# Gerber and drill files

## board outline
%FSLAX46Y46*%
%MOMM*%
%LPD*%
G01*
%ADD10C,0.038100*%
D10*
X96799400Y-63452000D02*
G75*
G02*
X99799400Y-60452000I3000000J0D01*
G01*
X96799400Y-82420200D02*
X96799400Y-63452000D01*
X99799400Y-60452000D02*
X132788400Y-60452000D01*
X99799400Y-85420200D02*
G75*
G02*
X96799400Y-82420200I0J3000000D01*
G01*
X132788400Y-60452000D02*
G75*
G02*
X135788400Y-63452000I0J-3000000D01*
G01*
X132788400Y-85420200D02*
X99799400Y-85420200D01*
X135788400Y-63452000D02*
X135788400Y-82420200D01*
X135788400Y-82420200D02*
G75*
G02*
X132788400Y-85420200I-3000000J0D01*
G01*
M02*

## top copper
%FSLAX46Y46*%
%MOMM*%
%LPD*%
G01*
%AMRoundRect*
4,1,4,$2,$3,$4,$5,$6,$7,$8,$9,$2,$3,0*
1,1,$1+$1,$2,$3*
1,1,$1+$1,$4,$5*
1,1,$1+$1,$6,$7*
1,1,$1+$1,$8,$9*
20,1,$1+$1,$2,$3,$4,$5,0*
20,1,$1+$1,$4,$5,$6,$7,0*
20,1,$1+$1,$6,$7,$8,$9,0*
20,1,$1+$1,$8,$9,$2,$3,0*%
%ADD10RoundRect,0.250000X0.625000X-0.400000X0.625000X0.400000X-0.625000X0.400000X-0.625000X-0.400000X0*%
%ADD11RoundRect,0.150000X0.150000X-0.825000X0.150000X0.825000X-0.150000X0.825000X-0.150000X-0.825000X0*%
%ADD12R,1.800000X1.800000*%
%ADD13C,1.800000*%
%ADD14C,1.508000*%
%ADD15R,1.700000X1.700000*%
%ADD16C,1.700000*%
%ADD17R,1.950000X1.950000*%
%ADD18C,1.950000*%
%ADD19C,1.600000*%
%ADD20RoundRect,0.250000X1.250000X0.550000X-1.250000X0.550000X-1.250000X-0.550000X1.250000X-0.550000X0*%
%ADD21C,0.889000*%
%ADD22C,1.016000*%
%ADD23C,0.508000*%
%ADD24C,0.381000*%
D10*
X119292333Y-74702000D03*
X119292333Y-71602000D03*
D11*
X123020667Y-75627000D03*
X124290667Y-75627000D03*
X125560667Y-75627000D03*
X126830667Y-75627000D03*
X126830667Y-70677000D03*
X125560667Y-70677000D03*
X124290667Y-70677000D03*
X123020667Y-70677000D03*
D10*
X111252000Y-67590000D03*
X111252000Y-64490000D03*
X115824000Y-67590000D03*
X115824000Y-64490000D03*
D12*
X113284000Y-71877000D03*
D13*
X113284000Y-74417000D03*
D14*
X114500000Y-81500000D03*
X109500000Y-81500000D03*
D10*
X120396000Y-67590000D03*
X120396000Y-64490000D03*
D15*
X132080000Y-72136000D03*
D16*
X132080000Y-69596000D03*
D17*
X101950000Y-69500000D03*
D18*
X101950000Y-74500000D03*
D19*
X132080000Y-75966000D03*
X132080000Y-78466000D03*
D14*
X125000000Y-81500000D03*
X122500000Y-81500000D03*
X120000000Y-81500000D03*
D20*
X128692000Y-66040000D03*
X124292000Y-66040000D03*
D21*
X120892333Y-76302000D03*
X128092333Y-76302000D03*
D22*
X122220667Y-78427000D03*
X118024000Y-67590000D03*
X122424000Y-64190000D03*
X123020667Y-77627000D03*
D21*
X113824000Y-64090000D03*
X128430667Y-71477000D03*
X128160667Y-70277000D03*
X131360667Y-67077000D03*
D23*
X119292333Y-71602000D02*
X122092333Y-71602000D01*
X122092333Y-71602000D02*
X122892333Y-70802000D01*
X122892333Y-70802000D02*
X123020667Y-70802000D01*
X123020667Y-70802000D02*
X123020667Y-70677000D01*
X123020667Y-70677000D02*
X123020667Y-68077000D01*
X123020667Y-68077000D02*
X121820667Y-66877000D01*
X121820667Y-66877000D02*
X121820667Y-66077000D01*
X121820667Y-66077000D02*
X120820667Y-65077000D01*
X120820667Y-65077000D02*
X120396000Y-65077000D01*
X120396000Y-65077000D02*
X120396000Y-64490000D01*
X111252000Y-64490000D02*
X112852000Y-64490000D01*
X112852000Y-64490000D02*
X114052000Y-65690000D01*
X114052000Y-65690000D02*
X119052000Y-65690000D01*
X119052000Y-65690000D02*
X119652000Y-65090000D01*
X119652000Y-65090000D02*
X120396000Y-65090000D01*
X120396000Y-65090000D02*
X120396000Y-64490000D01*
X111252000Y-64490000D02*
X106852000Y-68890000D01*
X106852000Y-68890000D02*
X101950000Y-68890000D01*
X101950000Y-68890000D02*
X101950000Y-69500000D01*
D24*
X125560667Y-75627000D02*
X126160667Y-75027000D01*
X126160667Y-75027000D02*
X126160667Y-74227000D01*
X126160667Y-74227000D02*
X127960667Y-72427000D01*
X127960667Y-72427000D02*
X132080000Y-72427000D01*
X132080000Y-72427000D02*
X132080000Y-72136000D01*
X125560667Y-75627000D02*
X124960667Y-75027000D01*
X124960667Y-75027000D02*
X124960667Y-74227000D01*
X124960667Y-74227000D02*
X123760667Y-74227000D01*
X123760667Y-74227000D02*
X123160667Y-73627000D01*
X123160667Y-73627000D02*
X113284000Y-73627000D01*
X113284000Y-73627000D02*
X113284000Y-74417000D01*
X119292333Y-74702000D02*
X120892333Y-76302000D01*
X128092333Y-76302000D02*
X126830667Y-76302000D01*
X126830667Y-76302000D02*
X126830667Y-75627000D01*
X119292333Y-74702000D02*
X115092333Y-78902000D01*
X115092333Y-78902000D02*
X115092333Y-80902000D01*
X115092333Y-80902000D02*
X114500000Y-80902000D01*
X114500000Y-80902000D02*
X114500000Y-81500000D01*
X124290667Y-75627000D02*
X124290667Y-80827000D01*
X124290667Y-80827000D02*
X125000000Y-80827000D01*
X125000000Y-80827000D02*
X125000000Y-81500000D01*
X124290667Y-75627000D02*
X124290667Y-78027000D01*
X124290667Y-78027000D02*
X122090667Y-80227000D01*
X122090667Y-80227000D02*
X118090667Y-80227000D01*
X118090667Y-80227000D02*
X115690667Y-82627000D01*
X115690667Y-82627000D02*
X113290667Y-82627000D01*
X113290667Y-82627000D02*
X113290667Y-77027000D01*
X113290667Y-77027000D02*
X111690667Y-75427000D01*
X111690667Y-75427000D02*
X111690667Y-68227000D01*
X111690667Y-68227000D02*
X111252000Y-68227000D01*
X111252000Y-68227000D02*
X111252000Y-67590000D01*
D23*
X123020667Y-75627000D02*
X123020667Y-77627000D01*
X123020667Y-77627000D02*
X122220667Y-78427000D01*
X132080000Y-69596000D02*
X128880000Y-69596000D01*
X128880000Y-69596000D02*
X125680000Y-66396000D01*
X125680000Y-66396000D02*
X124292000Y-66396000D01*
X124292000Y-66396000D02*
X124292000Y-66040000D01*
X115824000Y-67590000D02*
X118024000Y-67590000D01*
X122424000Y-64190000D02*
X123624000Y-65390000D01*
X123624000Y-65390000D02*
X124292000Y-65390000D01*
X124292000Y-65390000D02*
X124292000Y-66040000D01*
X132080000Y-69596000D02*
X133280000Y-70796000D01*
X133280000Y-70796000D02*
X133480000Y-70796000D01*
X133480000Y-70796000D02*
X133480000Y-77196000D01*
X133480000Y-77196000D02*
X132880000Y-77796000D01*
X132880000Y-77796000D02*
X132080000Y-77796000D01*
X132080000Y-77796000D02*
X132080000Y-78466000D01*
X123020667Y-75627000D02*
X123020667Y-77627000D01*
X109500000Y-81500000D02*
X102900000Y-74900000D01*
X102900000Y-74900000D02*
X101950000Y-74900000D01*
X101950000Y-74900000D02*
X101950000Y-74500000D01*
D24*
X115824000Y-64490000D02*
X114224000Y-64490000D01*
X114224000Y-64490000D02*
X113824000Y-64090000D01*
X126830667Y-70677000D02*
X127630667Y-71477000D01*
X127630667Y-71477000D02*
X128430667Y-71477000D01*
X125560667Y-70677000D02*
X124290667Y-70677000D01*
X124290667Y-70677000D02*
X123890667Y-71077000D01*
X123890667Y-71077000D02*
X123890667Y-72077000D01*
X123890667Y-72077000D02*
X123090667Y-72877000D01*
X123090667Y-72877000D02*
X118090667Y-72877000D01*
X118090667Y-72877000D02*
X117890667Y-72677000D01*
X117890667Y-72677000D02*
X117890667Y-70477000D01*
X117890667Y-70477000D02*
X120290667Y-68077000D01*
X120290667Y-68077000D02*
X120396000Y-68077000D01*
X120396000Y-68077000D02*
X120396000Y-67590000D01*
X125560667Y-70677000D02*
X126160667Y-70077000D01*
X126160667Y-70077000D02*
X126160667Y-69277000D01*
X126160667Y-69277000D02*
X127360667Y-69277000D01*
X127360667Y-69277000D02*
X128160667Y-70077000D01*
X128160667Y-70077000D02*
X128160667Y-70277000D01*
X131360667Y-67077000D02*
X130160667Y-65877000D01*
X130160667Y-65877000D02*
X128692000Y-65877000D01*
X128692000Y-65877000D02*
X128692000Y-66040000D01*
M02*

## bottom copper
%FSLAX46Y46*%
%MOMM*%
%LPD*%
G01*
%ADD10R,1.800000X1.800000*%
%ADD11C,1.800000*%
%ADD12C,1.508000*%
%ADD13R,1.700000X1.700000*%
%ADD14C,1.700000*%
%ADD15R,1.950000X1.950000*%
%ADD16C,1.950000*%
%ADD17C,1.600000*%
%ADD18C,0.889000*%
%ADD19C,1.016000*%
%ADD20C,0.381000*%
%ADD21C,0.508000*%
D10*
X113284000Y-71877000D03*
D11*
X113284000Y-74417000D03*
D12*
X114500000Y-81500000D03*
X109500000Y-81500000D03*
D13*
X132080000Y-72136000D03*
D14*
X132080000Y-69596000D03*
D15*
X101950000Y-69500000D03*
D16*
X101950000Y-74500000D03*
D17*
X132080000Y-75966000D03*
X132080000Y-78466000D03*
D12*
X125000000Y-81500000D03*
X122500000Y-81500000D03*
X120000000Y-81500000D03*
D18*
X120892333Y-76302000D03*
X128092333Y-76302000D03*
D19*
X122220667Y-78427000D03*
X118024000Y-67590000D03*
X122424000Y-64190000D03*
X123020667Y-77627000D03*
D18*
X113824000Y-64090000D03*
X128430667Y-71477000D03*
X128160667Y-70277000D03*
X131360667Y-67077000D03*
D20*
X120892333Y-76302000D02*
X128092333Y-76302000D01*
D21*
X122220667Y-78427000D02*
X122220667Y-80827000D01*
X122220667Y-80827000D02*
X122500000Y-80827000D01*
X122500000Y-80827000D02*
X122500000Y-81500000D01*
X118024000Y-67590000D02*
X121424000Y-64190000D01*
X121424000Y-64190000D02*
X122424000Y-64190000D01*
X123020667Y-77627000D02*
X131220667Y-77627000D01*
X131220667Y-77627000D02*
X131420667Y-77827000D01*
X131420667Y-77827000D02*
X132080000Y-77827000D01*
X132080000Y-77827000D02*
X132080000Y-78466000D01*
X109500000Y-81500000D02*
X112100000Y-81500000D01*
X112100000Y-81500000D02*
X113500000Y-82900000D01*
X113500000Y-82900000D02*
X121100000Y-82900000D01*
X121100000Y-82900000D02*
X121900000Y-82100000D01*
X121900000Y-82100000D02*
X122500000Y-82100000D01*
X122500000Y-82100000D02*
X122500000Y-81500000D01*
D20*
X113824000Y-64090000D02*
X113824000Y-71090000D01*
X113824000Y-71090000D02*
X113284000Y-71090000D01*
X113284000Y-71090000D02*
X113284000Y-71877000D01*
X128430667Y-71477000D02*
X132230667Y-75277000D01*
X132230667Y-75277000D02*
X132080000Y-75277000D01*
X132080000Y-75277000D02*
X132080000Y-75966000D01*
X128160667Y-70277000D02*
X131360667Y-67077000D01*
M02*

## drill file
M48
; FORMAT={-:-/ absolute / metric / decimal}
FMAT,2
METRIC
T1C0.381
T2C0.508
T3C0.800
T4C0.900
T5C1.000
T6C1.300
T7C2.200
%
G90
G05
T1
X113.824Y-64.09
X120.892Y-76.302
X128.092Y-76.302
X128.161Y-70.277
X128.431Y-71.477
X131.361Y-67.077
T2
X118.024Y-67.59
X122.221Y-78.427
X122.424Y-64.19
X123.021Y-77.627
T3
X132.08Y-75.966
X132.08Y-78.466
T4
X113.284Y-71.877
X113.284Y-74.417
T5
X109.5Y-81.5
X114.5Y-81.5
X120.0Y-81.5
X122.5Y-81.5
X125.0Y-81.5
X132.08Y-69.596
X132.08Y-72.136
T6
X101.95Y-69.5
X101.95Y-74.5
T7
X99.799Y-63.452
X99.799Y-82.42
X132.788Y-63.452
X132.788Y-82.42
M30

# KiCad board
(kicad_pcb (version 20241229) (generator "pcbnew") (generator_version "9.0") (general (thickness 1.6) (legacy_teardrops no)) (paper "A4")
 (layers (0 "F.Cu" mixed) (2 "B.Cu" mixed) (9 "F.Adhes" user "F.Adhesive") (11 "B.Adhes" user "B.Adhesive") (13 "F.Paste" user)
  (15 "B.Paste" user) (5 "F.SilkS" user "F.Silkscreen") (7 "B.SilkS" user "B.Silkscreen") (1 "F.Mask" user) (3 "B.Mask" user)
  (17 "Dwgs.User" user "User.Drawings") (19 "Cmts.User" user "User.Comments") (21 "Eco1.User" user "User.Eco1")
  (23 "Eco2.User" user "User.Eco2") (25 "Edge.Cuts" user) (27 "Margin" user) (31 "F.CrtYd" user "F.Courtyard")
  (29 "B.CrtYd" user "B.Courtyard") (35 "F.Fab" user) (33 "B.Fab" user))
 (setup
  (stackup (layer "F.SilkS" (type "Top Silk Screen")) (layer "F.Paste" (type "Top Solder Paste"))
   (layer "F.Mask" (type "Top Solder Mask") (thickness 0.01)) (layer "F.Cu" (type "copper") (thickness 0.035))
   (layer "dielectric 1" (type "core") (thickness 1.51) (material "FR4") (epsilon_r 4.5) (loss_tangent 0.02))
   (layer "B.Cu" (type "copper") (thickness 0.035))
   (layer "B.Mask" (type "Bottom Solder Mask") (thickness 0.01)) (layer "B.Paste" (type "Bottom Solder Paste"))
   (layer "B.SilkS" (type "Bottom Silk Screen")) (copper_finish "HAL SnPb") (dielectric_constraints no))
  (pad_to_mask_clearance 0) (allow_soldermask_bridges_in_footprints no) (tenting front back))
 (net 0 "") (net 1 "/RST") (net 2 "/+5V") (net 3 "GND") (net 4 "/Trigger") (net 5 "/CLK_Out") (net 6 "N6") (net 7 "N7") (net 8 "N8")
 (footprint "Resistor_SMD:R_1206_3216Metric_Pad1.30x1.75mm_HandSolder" (layer "F.Cu") (at 119.292333 73.152 90)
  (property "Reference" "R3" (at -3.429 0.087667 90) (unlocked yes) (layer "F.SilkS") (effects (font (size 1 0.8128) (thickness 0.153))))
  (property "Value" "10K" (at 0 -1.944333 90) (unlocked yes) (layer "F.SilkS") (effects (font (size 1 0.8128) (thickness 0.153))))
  (pad "1" smd roundrect (at -1.55 0 90) (size 1.3 1.75) (layers "F.Cu" "F.Mask" "F.Paste") (roundrect_rratio 0.192308) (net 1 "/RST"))
  (pad "2" smd roundrect (at 1.55 0 90) (size 1.3 1.75) (layers "F.Cu" "F.Mask" "F.Paste") (roundrect_rratio 0.192308) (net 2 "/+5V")))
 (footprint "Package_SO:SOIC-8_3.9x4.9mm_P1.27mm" (layer "F.Cu") (at 124.925667 73.152 90)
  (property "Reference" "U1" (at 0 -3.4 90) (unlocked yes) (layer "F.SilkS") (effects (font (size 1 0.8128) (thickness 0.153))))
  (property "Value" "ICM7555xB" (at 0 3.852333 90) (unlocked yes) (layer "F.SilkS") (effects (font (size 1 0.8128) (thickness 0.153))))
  (pad "1" smd roundrect (at -2.475 -1.905 90) (size 1.95 0.6) (layers "F.Cu" "F.Mask" "F.Paste") (roundrect_rratio 0.25) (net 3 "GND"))
  (pad "2" smd roundrect (at -2.475 -0.635 90) (size 1.95 0.6) (layers "F.Cu" "F.Mask" "F.Paste") (roundrect_rratio 0.25) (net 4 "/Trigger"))
  (pad "3" smd roundrect (at -2.475 0.635 90) (size 1.95 0.6) (layers "F.Cu" "F.Mask" "F.Paste") (roundrect_rratio 0.25) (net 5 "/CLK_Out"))
  (pad "4" smd roundrect (at -2.475 1.905 90) (size 1.95 0.6) (layers "F.Cu" "F.Mask" "F.Paste") (roundrect_rratio 0.25) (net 1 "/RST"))
  (pad "5" smd roundrect (at 2.475 1.905 90) (size 1.95 0.6) (layers "F.Cu" "F.Mask" "F.Paste") (roundrect_rratio 0.25) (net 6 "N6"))
  (pad "6" smd roundrect (at 2.475 0.635 90) (size 1.95 0.6) (layers "F.Cu" "F.Mask" "F.Paste") (roundrect_rratio 0.25) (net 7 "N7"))
  (pad "7" smd roundrect (at 2.475 -0.635 90) (size 1.95 0.6) (layers "F.Cu" "F.Mask" "F.Paste") (roundrect_rratio 0.25) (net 7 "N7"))
  (pad "8" smd roundrect (at 2.475 -1.905 90) (size 1.95 0.6) (layers "F.Cu" "F.Mask" "F.Paste") (roundrect_rratio 0.25) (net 2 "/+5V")))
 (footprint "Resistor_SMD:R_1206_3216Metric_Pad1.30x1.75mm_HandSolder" (layer "F.Cu") (at 111.252 66.04 90)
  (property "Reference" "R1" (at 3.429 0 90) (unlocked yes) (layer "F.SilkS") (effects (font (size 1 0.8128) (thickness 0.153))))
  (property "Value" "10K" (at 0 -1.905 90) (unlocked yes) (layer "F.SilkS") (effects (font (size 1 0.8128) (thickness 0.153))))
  (pad "1" smd roundrect (at -1.55 0 90) (size 1.3 1.75) (layers "F.Cu" "F.Mask" "F.Paste") (roundrect_rratio 0.192308) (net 4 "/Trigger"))
  (pad "2" smd roundrect (at 1.55 0 90) (size 1.3 1.75) (layers "F.Cu" "F.Mask" "F.Paste") (roundrect_rratio 0.192308) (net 2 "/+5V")))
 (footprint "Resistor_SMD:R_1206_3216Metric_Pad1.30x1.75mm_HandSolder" (layer "F.Cu") (at 115.824 66.04 90)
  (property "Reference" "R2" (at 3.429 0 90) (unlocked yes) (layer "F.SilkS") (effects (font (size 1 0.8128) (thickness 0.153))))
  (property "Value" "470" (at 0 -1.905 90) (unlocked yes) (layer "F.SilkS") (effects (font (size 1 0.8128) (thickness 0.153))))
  (pad "1" smd roundrect (at -1.55 0 90) (size 1.3 1.75) (layers "F.Cu" "F.Mask" "F.Paste") (roundrect_rratio 0.192308) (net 3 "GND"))
  (pad "2" smd roundrect (at 1.55 0 90) (size 1.3 1.75) (layers "F.Cu" "F.Mask" "F.Paste") (roundrect_rratio 0.192308) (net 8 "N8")))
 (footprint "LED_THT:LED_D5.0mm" (layer "F.Cu") (at 113.284 71.877 -90)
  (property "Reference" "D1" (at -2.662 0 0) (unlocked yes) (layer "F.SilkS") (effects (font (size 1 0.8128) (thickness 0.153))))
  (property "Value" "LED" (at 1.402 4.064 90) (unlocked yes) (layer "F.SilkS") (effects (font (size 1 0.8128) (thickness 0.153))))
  (pad "1" thru_hole rect (at 0 0 270) (size 1.8 1.8) (drill 0.9) (layers "*.Cu" "*.Mask") (remove_unused_layers no) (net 8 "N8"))
  (pad "2" thru_hole circle (at 2.54 0 270) (size 1.8 1.8) (drill 0.9) (layers "*.Cu" "*.Mask") (remove_unused_layers no) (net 5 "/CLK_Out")))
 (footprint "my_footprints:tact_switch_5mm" (layer "F.Cu") (at 112 81.5 180)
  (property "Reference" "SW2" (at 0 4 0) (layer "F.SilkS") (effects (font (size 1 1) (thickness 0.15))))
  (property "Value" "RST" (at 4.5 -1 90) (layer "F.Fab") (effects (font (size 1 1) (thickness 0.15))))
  (pad "1" thru_hole circle (at -2.5 0 180) (size 1.508 1.508) (drill 1) (layers "*.Cu" "*.Mask") (remove_unused_layers no) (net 1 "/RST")
   (solder_mask_margin 0.102))
  (pad "2" thru_hole circle (at 2.5 0 180) (size 1.508 1.508) (drill 1) (layers "*.Cu" "*.Mask") (remove_unused_layers no) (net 3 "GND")
   (solder_mask_margin 0.102)))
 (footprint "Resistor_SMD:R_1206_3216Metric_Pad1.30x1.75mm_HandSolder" (layer "F.Cu") (at 120.396 66.04 90)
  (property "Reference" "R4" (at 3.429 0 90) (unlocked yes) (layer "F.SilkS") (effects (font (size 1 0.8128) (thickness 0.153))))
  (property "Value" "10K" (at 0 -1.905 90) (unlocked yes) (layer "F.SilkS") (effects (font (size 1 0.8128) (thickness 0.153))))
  (pad "1" smd roundrect (at -1.55 0 90) (size 1.3 1.75) (layers "F.Cu" "F.Mask" "F.Paste") (roundrect_rratio 0.192308) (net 7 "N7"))
  (pad "2" smd roundrect (at 1.55 0 90) (size 1.3 1.75) (layers "F.Cu" "F.Mask" "F.Paste") (roundrect_rratio 0.192308) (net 2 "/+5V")))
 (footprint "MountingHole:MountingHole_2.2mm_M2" (layer "F.Cu") (at 99.7994 63.452)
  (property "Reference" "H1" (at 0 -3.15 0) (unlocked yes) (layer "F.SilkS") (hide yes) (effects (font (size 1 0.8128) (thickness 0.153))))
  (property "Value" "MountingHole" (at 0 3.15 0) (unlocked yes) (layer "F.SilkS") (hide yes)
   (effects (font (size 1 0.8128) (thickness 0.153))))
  (pad "" np_thru_hole circle (at 0 0) (size 2.2 2.2) (drill 2.2) (layers "*.Cu" "*.Mask")))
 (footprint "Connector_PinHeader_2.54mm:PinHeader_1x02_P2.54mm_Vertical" (layer "F.Cu") (at 132.08 72.136 180)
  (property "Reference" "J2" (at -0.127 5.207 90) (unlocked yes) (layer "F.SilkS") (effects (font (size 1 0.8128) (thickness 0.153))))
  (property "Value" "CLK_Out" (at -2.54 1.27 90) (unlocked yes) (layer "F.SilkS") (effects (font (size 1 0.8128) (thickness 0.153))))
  (pad "1" thru_hole rect (at 0 0 180) (size 1.7 1.7) (drill 1) (layers "*.Cu" "*.Mask") (remove_unused_layers no) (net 5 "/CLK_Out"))
  (pad "2" thru_hole circle (at 0 2.54 180) (size 1.7 1.7) (drill 1) (layers "*.Cu" "*.Mask") (remove_unused_layers no) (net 3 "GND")))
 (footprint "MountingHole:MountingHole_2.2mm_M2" (layer "F.Cu") (at 132.7884 82.4202)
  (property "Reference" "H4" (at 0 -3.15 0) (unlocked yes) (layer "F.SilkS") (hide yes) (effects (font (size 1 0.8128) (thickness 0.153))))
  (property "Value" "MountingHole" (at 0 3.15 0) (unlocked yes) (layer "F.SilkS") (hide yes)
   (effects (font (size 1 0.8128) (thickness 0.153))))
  (pad "" np_thru_hole circle (at 0 0) (size 2.2 2.2) (drill 2.2) (layers "*.Cu" "*.Mask")))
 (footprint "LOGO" (layer "F.Cu") (at 105.5 63.5)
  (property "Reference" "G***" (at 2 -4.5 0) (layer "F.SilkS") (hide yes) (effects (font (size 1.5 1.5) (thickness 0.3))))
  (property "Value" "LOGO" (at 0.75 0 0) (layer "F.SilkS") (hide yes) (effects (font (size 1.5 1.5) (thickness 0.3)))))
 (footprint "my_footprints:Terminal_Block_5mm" (layer "F.Cu") (at 101.95 72 -90)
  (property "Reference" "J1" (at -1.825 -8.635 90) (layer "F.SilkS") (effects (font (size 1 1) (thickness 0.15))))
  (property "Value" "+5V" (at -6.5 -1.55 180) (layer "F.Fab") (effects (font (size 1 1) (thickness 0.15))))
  (pad "1" thru_hole rect (at -2.5 0 270) (size 1.95 1.95) (drill 1.3) (layers "*.Cu" "*.Mask") (remove_unused_layers no) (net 2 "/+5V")
   (solder_mask_margin 0.102))
  (pad "2" thru_hole circle (at 2.5 0 270) (size 1.95 1.95) (drill 1.3) (layers "*.Cu" "*.Mask") (remove_unused_layers no) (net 3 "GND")
   (solder_mask_margin 0.102)))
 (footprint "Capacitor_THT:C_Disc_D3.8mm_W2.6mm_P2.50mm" (layer "F.Cu") (at 132.08 75.966 -90)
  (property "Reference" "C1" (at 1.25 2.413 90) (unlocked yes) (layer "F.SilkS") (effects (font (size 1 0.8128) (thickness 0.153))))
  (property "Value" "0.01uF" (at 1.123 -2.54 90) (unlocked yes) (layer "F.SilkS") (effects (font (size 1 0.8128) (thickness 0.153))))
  (pad "1" thru_hole circle (at 0 0 270) (size 1.6 1.6) (drill 0.8) (layers "*.Cu" "*.Mask") (remove_unused_layers no) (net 6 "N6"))
  (pad "2" thru_hole circle (at 2.5 0 270) (size 1.6 1.6) (drill 0.8) (layers "*.Cu" "*.Mask") (remove_unused_layers no) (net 3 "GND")))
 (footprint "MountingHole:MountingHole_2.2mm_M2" (layer "F.Cu") (at 132.7884 63.452)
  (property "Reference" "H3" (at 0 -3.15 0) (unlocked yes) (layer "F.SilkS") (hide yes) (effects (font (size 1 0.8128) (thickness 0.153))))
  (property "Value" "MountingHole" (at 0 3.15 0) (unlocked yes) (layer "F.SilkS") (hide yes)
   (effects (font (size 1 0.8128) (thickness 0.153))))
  (pad "" np_thru_hole circle (at 0 0) (size 2.2 2.2) (drill 2.2) (layers "*.Cu" "*.Mask")))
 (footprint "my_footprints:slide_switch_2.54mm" (layer "F.Cu") (at 122.5 81.5 180)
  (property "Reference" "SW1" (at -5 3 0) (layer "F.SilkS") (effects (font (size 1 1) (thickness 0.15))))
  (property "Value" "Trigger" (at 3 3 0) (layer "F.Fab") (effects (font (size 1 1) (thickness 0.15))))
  (pad "1" thru_hole circle (at -2.5 0 180) (size 1.508 1.508) (drill 1) (layers "*.Cu" "*.Mask") (remove_unused_layers no)
   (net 4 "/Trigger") (solder_mask_margin 0.102))
  (pad "2" thru_hole circle (at 0 0 180) (size 1.508 1.508) (drill 1) (layers "*.Cu" "*.Mask") (remove_unused_layers no) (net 3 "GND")
   (solder_mask_margin 0.102))
  (pad "3" thru_hole circle (at 2.5 0 180) (size 1.508 1.508) (drill 1) (layers "*.Cu" "*.Mask") (remove_unused_layers no)
   (solder_mask_margin 0.102)))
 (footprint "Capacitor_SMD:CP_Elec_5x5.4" (layer "F.Cu") (at 126.492 66.04 180)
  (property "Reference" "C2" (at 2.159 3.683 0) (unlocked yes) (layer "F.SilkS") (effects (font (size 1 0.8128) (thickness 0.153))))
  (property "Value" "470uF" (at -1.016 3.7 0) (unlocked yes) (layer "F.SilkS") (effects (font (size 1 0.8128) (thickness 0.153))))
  (pad "1" smd roundrect (at -2.2 0 180) (size 3 1.6) (layers "F.Cu" "F.Mask" "F.Paste") (roundrect_rratio 0.15625) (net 7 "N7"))
  (pad "2" smd roundrect (at 2.2 0 180) (size 3 1.6) (layers "F.Cu" "F.Mask" "F.Paste") (roundrect_rratio 0.15625) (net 3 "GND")))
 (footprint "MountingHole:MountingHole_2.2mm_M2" (layer "F.Cu") (at 99.7994 82.4202)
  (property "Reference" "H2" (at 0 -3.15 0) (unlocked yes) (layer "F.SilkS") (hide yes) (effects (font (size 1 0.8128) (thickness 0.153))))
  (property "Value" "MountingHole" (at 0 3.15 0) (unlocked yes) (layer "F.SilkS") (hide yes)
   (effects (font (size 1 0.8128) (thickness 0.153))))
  (pad "" np_thru_hole circle (at 0 0) (size 2.2 2.2) (drill 2.2) (layers "*.Cu" "*.Mask")))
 (gr_arc (start 96.7994 63.452) (mid 97.67808 61.33068) (end 99.7994 60.452) (stroke (width 0.0381) (type default)) (layer "Edge.Cuts"))
 (gr_line (start 96.7994 82.4202) (end 96.7994 63.452) (stroke (width 0.0381) (type default)) (layer "Edge.Cuts"))
 (gr_line (start 99.7994 60.452) (end 132.7884 60.452) (stroke (width 0.0381) (type default)) (layer "Edge.Cuts"))
 (gr_arc (start 99.7994 85.4202) (mid 97.67808 84.54152) (end 96.7994 82.4202) (stroke (width 0.0381) (type default)) (layer "Edge.Cuts"))
 (gr_arc (start 132.7884 60.452) (mid 134.90972 61.33068) (end 135.7884 63.452) (stroke (width 0.0381) (type default)) (layer "Edge.Cuts"))
 (gr_line (start 132.7884 85.4202) (end 99.7994 85.4202) (stroke (width 0.0381) (type default)) (layer "Edge.Cuts"))
 (gr_line (start 135.7884 63.452) (end 135.7884 82.4202) (stroke (width 0.0381) (type default)) (layer "Edge.Cuts"))
 (gr_arc (start 135.7884 82.4202) (mid 134.90972 84.54152) (end 132.7884 85.4202) (stroke (width 0.0381) (type default)) (layer "Edge.Cuts"))
 (segment (start 119.292333 71.602000) (end 122.092333 71.602000) (width 0.508000) (layer "F.Cu") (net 2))
 (segment (start 122.092333 71.602000) (end 122.892333 70.802000) (width 0.508000) (layer "F.Cu") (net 2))
 (segment (start 122.892333 70.802000) (end 123.020667 70.802000) (width 0.508000) (layer "F.Cu") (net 2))
 (segment (start 123.020667 70.802000) (end 123.020667 70.677000) (width 0.508000) (layer "F.Cu") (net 2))
 (segment (start 123.020667 70.677000) (end 123.020667 68.077000) (width 0.508000) (layer "F.Cu") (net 2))
 (segment (start 123.020667 68.077000) (end 121.820667 66.877000) (width 0.508000) (layer "F.Cu") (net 2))
 (segment (start 121.820667 66.877000) (end 121.820667 66.077000) (width 0.508000) (layer "F.Cu") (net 2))
 (segment (start 121.820667 66.077000) (end 120.820667 65.077000) (width 0.508000) (layer "F.Cu") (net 2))
 (segment (start 120.820667 65.077000) (end 120.396000 65.077000) (width 0.508000) (layer "F.Cu") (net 2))
 (segment (start 120.396000 65.077000) (end 120.396000 64.490000) (width 0.508000) (layer "F.Cu") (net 2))
 (segment (start 111.252000 64.490000) (end 112.852000 64.490000) (width 0.508000) (layer "F.Cu") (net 2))
 (segment (start 112.852000 64.490000) (end 114.052000 65.690000) (width 0.508000) (layer "F.Cu") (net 2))
 (segment (start 114.052000 65.690000) (end 119.052000 65.690000) (width 0.508000) (layer "F.Cu") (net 2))
 (segment (start 119.052000 65.690000) (end 119.652000 65.090000) (width 0.508000) (layer "F.Cu") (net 2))
 (segment (start 119.652000 65.090000) (end 120.396000 65.090000) (width 0.508000) (layer "F.Cu") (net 2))
 (segment (start 120.396000 65.090000) (end 120.396000 64.490000) (width 0.508000) (layer "F.Cu") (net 2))
 (segment (start 111.252000 64.490000) (end 106.852000 68.890000) (width 0.508000) (layer "F.Cu") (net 2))
 (segment (start 106.852000 68.890000) (end 101.950000 68.890000) (width 0.508000) (layer "F.Cu") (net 2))
 (segment (start 101.950000 68.890000) (end 101.950000 69.500000) (width 0.508000) (layer "F.Cu") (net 2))
 (segment (start 125.560667 75.627000) (end 126.160667 75.027000) (width 0.381000) (layer "F.Cu") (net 5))
 (segment (start 126.160667 75.027000) (end 126.160667 74.227000) (width 0.381000) (layer "F.Cu") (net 5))
 (segment (start 126.160667 74.227000) (end 127.960667 72.427000) (width 0.381000) (layer "F.Cu") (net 5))
 (segment (start 127.960667 72.427000) (end 132.080000 72.427000) (width 0.381000) (layer "F.Cu") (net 5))
 (segment (start 132.080000 72.427000) (end 132.080000 72.136000) (width 0.381000) (layer "F.Cu") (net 5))
 (segment (start 125.560667 75.627000) (end 124.960667 75.027000) (width 0.381000) (layer "F.Cu") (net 5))
 (segment (start 124.960667 75.027000) (end 124.960667 74.227000) (width 0.381000) (layer "F.Cu") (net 5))
 (segment (start 124.960667 74.227000) (end 123.760667 74.227000) (width 0.381000) (layer "F.Cu") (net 5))
 (segment (start 123.760667 74.227000) (end 123.160667 73.627000) (width 0.381000) (layer "F.Cu") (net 5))
 (segment (start 123.160667 73.627000) (end 113.284000 73.627000) (width 0.381000) (layer "F.Cu") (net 5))
 (segment (start 113.284000 73.627000) (end 113.284000 74.417000) (width 0.381000) (layer "F.Cu") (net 5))
 (segment (start 119.292333 74.702000) (end 120.892333 76.302000) (width 0.381000) (layer "F.Cu") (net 1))
 (segment (start 120.892333 76.302000) (end 128.092333 76.302000) (width 0.381000) (layer "B.Cu") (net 1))
 (segment (start 128.092333 76.302000) (end 126.830667 76.302000) (width 0.381000) (layer "F.Cu") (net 1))
 (segment (start 126.830667 76.302000) (end 126.830667 75.627000) (width 0.381000) (layer "F.Cu") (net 1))
 (segment (start 119.292333 74.702000) (end 115.092333 78.902000) (width 0.381000) (layer "F.Cu") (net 1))
 (segment (start 115.092333 78.902000) (end 115.092333 80.902000) (width 0.381000) (layer "F.Cu") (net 1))
 (segment (start 115.092333 80.902000) (end 114.500000 80.902000) (width 0.381000) (layer "F.Cu") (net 1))
 (segment (start 114.500000 80.902000) (end 114.500000 81.500000) (width 0.381000) (layer "F.Cu") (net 1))
 (segment (start 124.290667 75.627000) (end 124.290667 80.827000) (width 0.381000) (layer "F.Cu") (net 4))
 (segment (start 124.290667 80.827000) (end 125.000000 80.827000) (width 0.381000) (layer "F.Cu") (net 4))
 (segment (start 125.000000 80.827000) (end 125.000000 81.500000) (width 0.381000) (layer "F.Cu") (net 4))
 (segment (start 124.290667 75.627000) (end 124.290667 78.027000) (width 0.381000) (layer "F.Cu") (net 4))
 (segment (start 124.290667 78.027000) (end 122.090667 80.227000) (width 0.381000) (layer "F.Cu") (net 4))
 (segment (start 122.090667 80.227000) (end 118.090667 80.227000) (width 0.381000) (layer "F.Cu") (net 4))
 (segment (start 118.090667 80.227000) (end 115.690667 82.627000) (width 0.381000) (layer "F.Cu") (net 4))
 (segment (start 115.690667 82.627000) (end 113.290667 82.627000) (width 0.381000) (layer "F.Cu") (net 4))
 (segment (start 113.290667 82.627000) (end 113.290667 77.027000) (width 0.381000) (layer "F.Cu") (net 4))
 (segment (start 113.290667 77.027000) (end 111.690667 75.427000) (width 0.381000) (layer "F.Cu") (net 4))
 (segment (start 111.690667 75.427000) (end 111.690667 68.227000) (width 0.381000) (layer "F.Cu") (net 4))
 (segment (start 111.690667 68.227000) (end 111.252000 68.227000) (width 0.381000) (layer "F.Cu") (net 4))
 (segment (start 111.252000 68.227000) (end 111.252000 67.590000) (width 0.381000) (layer "F.Cu") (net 4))
 (segment (start 123.020667 75.627000) (end 123.020667 77.627000) (width 0.508000) (layer "F.Cu") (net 3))
 (segment (start 123.020667 77.627000) (end 122.220667 78.427000) (width 0.508000) (layer "F.Cu") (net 3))
 (segment (start 122.220667 78.427000) (end 122.220667 80.827000) (width 0.508000) (layer "B.Cu") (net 3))
 (segment (start 122.220667 80.827000) (end 122.500000 80.827000) (width 0.508000) (layer "B.Cu") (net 3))
 (segment (start 122.500000 80.827000) (end 122.500000 81.500000) (width 0.508000) (layer "B.Cu") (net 3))
 (segment (start 132.080000 69.596000) (end 128.880000 69.596000) (width 0.508000) (layer "F.Cu") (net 3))
 (segment (start 128.880000 69.596000) (end 125.680000 66.396000) (width 0.508000) (layer "F.Cu") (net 3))
 (segment (start 125.680000 66.396000) (end 124.292000 66.396000) (width 0.508000) (layer "F.Cu") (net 3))
 (segment (start 124.292000 66.396000) (end 124.292000 66.040000) (width 0.508000) (layer "F.Cu") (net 3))
 (segment (start 115.824000 67.590000) (end 118.024000 67.590000) (width 0.508000) (layer "F.Cu") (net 3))
 (segment (start 118.024000 67.590000) (end 121.424000 64.190000) (width 0.508000) (layer "B.Cu") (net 3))
 (segment (start 121.424000 64.190000) (end 122.424000 64.190000) (width 0.508000) (layer "B.Cu") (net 3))
 (segment (start 122.424000 64.190000) (end 123.624000 65.390000) (width 0.508000) (layer "F.Cu") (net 3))
 (segment (start 123.624000 65.390000) (end 124.292000 65.390000) (width 0.508000) (layer "F.Cu") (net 3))
 (segment (start 124.292000 65.390000) (end 124.292000 66.040000) (width 0.508000) (layer "F.Cu") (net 3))
 (segment (start 132.080000 69.596000) (end 133.280000 70.796000) (width 0.508000) (layer "F.Cu") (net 3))
 (segment (start 133.280000 70.796000) (end 133.480000 70.796000) (width 0.508000) (layer "F.Cu") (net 3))
 (segment (start 133.480000 70.796000) (end 133.480000 77.196000) (width 0.508000) (layer "F.Cu") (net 3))
 (segment (start 133.480000 77.196000) (end 132.880000 77.796000) (width 0.508000) (layer "F.Cu") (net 3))
 (segment (start 132.880000 77.796000) (end 132.080000 77.796000) (width 0.508000) (layer "F.Cu") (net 3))
 (segment (start 132.080000 77.796000) (end 132.080000 78.466000) (width 0.508000) (layer "F.Cu") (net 3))
 (segment (start 123.020667 75.627000) (end 123.020667 77.627000) (width 0.508000) (layer "F.Cu") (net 3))
 (segment (start 123.020667 77.627000) (end 131.220667 77.627000) (width 0.508000) (layer "B.Cu") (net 3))
 (segment (start 131.220667 77.627000) (end 131.420667 77.827000) (width 0.508000) (layer "B.Cu") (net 3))
 (segment (start 131.420667 77.827000) (end 132.080000 77.827000) (width 0.508000) (layer "B.Cu") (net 3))
 (segment (start 132.080000 77.827000) (end 132.080000 78.466000) (width 0.508000) (layer "B.Cu") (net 3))
 (segment (start 109.500000 81.500000) (end 102.900000 74.900000) (width 0.508000) (layer "F.Cu") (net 3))
 (segment (start 102.900000 74.900000) (end 101.950000 74.900000) (width 0.508000) (layer "F.Cu") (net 3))
 (segment (start 101.950000 74.900000) (end 101.950000 74.500000) (width 0.508000) (layer "F.Cu") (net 3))
 (segment (start 109.500000 81.500000) (end 112.100000 81.500000) (width 0.508000) (layer "B.Cu") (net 3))
 (segment (start 112.100000 81.500000) (end 113.500000 82.900000) (width 0.508000) (layer "B.Cu") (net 3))
 (segment (start 113.500000 82.900000) (end 121.100000 82.900000) (width 0.508000) (layer "B.Cu") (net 3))
 (segment (start 121.100000 82.900000) (end 121.900000 82.100000) (width 0.508000) (layer "B.Cu") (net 3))
 (segment (start 121.900000 82.100000) (end 122.500000 82.100000) (width 0.508000) (layer "B.Cu") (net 3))
 (segment (start 122.500000 82.100000) (end 122.500000 81.500000) (width 0.508000) (layer "B.Cu") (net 3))
 (segment (start 115.824000 64.490000) (end 114.224000 64.490000) (width 0.381000) (layer "F.Cu") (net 8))
 (segment (start 114.224000 64.490000) (end 113.824000 64.090000) (width 0.381000) (layer "F.Cu") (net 8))
 (segment (start 113.824000 64.090000) (end 113.824000 71.090000) (width 0.381000) (layer "B.Cu") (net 8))
 (segment (start 113.824000 71.090000) (end 113.284000 71.090000) (width 0.381000) (layer "B.Cu") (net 8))
 (segment (start 113.284000 71.090000) (end 113.284000 71.877000) (width 0.381000) (layer "B.Cu") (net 8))
 (segment (start 126.830667 70.677000) (end 127.630667 71.477000) (width 0.381000) (layer "F.Cu") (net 6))
 (segment (start 127.630667 71.477000) (end 128.430667 71.477000) (width 0.381000) (layer "F.Cu") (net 6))
 (segment (start 128.430667 71.477000) (end 132.230667 75.277000) (width 0.381000) (layer "B.Cu") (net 6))
 (segment (start 132.230667 75.277000) (end 132.080000 75.277000) (width 0.381000) (layer "B.Cu") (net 6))
 (segment (start 132.080000 75.277000) (end 132.080000 75.966000) (width 0.381000) (layer "B.Cu") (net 6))
 (segment (start 125.560667 70.677000) (end 124.290667 70.677000) (width 0.381000) (layer "F.Cu") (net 7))
 (segment (start 124.290667 70.677000) (end 123.890667 71.077000) (width 0.381000) (layer "F.Cu") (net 7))
 (segment (start 123.890667 71.077000) (end 123.890667 72.077000) (width 0.381000) (layer "F.Cu") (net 7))
 (segment (start 123.890667 72.077000) (end 123.090667 72.877000) (width 0.381000) (layer "F.Cu") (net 7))
 (segment (start 123.090667 72.877000) (end 118.090667 72.877000) (width 0.381000) (layer "F.Cu") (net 7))
 (segment (start 118.090667 72.877000) (end 117.890667 72.677000) (width 0.381000) (layer "F.Cu") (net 7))
 (segment (start 117.890667 72.677000) (end 117.890667 70.477000) (width 0.381000) (layer "F.Cu") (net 7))
 (segment (start 117.890667 70.477000) (end 120.290667 68.077000) (width 0.381000) (layer "F.Cu") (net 7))
 (segment (start 120.290667 68.077000) (end 120.396000 68.077000) (width 0.381000) (layer "F.Cu") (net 7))
 (segment (start 120.396000 68.077000) (end 120.396000 67.590000) (width 0.381000) (layer "F.Cu") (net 7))
 (segment (start 125.560667 70.677000) (end 126.160667 70.077000) (width 0.381000) (layer "F.Cu") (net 7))
 (segment (start 126.160667 70.077000) (end 126.160667 69.277000) (width 0.381000) (layer "F.Cu") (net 7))
 (segment (start 126.160667 69.277000) (end 127.360667 69.277000) (width 0.381000) (layer "F.Cu") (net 7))
 (segment (start 127.360667 69.277000) (end 128.160667 70.077000) (width 0.381000) (layer "F.Cu") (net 7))
 (segment (start 128.160667 70.077000) (end 128.160667 70.277000) (width 0.381000) (layer "F.Cu") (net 7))
 (segment (start 128.160667 70.277000) (end 131.360667 67.077000) (width 0.381000) (layer "B.Cu") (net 7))
 (segment (start 131.360667 67.077000) (end 130.160667 65.877000) (width 0.381000) (layer "F.Cu") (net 7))
 (segment (start 130.160667 65.877000) (end 128.692000 65.877000) (width 0.381000) (layer "F.Cu") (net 7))
 (segment (start 128.692000 65.877000) (end 128.692000 66.040000) (width 0.381000) (layer "F.Cu") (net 7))
 (via (at 120.892333 76.302000) (size 0.889000) (drill 0.381000) (layers "F.Cu" "B.Cu") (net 1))
 (via (at 128.092333 76.302000) (size 0.889000) (drill 0.381000) (layers "F.Cu" "B.Cu") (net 1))
 (via (at 122.220667 78.427000) (size 1.016000) (drill 0.508000) (layers "F.Cu" "B.Cu") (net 3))
 (via (at 118.024000 67.590000) (size 1.016000) (drill 0.508000) (layers "F.Cu" "B.Cu") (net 3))
 (via (at 122.424000 64.190000) (size 1.016000) (drill 0.508000) (layers "F.Cu" "B.Cu") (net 3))
 (via (at 123.020667 77.627000) (size 1.016000) (drill 0.508000) (layers "F.Cu" "B.Cu") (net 3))
 (via (at 113.824000 64.090000) (size 0.889000) (drill 0.381000) (layers "F.Cu" "B.Cu") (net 8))
 (via (at 128.430667 71.477000) (size 0.889000) (drill 0.381000) (layers "F.Cu" "B.Cu") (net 6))
 (via (at 128.160667 70.277000) (size 0.889000) (drill 0.381000) (layers "F.Cu" "B.Cu") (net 7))
 (via (at 131.360667 67.077000) (size 0.889000) (drill 0.381000) (layers "F.Cu" "B.Cu") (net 7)))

